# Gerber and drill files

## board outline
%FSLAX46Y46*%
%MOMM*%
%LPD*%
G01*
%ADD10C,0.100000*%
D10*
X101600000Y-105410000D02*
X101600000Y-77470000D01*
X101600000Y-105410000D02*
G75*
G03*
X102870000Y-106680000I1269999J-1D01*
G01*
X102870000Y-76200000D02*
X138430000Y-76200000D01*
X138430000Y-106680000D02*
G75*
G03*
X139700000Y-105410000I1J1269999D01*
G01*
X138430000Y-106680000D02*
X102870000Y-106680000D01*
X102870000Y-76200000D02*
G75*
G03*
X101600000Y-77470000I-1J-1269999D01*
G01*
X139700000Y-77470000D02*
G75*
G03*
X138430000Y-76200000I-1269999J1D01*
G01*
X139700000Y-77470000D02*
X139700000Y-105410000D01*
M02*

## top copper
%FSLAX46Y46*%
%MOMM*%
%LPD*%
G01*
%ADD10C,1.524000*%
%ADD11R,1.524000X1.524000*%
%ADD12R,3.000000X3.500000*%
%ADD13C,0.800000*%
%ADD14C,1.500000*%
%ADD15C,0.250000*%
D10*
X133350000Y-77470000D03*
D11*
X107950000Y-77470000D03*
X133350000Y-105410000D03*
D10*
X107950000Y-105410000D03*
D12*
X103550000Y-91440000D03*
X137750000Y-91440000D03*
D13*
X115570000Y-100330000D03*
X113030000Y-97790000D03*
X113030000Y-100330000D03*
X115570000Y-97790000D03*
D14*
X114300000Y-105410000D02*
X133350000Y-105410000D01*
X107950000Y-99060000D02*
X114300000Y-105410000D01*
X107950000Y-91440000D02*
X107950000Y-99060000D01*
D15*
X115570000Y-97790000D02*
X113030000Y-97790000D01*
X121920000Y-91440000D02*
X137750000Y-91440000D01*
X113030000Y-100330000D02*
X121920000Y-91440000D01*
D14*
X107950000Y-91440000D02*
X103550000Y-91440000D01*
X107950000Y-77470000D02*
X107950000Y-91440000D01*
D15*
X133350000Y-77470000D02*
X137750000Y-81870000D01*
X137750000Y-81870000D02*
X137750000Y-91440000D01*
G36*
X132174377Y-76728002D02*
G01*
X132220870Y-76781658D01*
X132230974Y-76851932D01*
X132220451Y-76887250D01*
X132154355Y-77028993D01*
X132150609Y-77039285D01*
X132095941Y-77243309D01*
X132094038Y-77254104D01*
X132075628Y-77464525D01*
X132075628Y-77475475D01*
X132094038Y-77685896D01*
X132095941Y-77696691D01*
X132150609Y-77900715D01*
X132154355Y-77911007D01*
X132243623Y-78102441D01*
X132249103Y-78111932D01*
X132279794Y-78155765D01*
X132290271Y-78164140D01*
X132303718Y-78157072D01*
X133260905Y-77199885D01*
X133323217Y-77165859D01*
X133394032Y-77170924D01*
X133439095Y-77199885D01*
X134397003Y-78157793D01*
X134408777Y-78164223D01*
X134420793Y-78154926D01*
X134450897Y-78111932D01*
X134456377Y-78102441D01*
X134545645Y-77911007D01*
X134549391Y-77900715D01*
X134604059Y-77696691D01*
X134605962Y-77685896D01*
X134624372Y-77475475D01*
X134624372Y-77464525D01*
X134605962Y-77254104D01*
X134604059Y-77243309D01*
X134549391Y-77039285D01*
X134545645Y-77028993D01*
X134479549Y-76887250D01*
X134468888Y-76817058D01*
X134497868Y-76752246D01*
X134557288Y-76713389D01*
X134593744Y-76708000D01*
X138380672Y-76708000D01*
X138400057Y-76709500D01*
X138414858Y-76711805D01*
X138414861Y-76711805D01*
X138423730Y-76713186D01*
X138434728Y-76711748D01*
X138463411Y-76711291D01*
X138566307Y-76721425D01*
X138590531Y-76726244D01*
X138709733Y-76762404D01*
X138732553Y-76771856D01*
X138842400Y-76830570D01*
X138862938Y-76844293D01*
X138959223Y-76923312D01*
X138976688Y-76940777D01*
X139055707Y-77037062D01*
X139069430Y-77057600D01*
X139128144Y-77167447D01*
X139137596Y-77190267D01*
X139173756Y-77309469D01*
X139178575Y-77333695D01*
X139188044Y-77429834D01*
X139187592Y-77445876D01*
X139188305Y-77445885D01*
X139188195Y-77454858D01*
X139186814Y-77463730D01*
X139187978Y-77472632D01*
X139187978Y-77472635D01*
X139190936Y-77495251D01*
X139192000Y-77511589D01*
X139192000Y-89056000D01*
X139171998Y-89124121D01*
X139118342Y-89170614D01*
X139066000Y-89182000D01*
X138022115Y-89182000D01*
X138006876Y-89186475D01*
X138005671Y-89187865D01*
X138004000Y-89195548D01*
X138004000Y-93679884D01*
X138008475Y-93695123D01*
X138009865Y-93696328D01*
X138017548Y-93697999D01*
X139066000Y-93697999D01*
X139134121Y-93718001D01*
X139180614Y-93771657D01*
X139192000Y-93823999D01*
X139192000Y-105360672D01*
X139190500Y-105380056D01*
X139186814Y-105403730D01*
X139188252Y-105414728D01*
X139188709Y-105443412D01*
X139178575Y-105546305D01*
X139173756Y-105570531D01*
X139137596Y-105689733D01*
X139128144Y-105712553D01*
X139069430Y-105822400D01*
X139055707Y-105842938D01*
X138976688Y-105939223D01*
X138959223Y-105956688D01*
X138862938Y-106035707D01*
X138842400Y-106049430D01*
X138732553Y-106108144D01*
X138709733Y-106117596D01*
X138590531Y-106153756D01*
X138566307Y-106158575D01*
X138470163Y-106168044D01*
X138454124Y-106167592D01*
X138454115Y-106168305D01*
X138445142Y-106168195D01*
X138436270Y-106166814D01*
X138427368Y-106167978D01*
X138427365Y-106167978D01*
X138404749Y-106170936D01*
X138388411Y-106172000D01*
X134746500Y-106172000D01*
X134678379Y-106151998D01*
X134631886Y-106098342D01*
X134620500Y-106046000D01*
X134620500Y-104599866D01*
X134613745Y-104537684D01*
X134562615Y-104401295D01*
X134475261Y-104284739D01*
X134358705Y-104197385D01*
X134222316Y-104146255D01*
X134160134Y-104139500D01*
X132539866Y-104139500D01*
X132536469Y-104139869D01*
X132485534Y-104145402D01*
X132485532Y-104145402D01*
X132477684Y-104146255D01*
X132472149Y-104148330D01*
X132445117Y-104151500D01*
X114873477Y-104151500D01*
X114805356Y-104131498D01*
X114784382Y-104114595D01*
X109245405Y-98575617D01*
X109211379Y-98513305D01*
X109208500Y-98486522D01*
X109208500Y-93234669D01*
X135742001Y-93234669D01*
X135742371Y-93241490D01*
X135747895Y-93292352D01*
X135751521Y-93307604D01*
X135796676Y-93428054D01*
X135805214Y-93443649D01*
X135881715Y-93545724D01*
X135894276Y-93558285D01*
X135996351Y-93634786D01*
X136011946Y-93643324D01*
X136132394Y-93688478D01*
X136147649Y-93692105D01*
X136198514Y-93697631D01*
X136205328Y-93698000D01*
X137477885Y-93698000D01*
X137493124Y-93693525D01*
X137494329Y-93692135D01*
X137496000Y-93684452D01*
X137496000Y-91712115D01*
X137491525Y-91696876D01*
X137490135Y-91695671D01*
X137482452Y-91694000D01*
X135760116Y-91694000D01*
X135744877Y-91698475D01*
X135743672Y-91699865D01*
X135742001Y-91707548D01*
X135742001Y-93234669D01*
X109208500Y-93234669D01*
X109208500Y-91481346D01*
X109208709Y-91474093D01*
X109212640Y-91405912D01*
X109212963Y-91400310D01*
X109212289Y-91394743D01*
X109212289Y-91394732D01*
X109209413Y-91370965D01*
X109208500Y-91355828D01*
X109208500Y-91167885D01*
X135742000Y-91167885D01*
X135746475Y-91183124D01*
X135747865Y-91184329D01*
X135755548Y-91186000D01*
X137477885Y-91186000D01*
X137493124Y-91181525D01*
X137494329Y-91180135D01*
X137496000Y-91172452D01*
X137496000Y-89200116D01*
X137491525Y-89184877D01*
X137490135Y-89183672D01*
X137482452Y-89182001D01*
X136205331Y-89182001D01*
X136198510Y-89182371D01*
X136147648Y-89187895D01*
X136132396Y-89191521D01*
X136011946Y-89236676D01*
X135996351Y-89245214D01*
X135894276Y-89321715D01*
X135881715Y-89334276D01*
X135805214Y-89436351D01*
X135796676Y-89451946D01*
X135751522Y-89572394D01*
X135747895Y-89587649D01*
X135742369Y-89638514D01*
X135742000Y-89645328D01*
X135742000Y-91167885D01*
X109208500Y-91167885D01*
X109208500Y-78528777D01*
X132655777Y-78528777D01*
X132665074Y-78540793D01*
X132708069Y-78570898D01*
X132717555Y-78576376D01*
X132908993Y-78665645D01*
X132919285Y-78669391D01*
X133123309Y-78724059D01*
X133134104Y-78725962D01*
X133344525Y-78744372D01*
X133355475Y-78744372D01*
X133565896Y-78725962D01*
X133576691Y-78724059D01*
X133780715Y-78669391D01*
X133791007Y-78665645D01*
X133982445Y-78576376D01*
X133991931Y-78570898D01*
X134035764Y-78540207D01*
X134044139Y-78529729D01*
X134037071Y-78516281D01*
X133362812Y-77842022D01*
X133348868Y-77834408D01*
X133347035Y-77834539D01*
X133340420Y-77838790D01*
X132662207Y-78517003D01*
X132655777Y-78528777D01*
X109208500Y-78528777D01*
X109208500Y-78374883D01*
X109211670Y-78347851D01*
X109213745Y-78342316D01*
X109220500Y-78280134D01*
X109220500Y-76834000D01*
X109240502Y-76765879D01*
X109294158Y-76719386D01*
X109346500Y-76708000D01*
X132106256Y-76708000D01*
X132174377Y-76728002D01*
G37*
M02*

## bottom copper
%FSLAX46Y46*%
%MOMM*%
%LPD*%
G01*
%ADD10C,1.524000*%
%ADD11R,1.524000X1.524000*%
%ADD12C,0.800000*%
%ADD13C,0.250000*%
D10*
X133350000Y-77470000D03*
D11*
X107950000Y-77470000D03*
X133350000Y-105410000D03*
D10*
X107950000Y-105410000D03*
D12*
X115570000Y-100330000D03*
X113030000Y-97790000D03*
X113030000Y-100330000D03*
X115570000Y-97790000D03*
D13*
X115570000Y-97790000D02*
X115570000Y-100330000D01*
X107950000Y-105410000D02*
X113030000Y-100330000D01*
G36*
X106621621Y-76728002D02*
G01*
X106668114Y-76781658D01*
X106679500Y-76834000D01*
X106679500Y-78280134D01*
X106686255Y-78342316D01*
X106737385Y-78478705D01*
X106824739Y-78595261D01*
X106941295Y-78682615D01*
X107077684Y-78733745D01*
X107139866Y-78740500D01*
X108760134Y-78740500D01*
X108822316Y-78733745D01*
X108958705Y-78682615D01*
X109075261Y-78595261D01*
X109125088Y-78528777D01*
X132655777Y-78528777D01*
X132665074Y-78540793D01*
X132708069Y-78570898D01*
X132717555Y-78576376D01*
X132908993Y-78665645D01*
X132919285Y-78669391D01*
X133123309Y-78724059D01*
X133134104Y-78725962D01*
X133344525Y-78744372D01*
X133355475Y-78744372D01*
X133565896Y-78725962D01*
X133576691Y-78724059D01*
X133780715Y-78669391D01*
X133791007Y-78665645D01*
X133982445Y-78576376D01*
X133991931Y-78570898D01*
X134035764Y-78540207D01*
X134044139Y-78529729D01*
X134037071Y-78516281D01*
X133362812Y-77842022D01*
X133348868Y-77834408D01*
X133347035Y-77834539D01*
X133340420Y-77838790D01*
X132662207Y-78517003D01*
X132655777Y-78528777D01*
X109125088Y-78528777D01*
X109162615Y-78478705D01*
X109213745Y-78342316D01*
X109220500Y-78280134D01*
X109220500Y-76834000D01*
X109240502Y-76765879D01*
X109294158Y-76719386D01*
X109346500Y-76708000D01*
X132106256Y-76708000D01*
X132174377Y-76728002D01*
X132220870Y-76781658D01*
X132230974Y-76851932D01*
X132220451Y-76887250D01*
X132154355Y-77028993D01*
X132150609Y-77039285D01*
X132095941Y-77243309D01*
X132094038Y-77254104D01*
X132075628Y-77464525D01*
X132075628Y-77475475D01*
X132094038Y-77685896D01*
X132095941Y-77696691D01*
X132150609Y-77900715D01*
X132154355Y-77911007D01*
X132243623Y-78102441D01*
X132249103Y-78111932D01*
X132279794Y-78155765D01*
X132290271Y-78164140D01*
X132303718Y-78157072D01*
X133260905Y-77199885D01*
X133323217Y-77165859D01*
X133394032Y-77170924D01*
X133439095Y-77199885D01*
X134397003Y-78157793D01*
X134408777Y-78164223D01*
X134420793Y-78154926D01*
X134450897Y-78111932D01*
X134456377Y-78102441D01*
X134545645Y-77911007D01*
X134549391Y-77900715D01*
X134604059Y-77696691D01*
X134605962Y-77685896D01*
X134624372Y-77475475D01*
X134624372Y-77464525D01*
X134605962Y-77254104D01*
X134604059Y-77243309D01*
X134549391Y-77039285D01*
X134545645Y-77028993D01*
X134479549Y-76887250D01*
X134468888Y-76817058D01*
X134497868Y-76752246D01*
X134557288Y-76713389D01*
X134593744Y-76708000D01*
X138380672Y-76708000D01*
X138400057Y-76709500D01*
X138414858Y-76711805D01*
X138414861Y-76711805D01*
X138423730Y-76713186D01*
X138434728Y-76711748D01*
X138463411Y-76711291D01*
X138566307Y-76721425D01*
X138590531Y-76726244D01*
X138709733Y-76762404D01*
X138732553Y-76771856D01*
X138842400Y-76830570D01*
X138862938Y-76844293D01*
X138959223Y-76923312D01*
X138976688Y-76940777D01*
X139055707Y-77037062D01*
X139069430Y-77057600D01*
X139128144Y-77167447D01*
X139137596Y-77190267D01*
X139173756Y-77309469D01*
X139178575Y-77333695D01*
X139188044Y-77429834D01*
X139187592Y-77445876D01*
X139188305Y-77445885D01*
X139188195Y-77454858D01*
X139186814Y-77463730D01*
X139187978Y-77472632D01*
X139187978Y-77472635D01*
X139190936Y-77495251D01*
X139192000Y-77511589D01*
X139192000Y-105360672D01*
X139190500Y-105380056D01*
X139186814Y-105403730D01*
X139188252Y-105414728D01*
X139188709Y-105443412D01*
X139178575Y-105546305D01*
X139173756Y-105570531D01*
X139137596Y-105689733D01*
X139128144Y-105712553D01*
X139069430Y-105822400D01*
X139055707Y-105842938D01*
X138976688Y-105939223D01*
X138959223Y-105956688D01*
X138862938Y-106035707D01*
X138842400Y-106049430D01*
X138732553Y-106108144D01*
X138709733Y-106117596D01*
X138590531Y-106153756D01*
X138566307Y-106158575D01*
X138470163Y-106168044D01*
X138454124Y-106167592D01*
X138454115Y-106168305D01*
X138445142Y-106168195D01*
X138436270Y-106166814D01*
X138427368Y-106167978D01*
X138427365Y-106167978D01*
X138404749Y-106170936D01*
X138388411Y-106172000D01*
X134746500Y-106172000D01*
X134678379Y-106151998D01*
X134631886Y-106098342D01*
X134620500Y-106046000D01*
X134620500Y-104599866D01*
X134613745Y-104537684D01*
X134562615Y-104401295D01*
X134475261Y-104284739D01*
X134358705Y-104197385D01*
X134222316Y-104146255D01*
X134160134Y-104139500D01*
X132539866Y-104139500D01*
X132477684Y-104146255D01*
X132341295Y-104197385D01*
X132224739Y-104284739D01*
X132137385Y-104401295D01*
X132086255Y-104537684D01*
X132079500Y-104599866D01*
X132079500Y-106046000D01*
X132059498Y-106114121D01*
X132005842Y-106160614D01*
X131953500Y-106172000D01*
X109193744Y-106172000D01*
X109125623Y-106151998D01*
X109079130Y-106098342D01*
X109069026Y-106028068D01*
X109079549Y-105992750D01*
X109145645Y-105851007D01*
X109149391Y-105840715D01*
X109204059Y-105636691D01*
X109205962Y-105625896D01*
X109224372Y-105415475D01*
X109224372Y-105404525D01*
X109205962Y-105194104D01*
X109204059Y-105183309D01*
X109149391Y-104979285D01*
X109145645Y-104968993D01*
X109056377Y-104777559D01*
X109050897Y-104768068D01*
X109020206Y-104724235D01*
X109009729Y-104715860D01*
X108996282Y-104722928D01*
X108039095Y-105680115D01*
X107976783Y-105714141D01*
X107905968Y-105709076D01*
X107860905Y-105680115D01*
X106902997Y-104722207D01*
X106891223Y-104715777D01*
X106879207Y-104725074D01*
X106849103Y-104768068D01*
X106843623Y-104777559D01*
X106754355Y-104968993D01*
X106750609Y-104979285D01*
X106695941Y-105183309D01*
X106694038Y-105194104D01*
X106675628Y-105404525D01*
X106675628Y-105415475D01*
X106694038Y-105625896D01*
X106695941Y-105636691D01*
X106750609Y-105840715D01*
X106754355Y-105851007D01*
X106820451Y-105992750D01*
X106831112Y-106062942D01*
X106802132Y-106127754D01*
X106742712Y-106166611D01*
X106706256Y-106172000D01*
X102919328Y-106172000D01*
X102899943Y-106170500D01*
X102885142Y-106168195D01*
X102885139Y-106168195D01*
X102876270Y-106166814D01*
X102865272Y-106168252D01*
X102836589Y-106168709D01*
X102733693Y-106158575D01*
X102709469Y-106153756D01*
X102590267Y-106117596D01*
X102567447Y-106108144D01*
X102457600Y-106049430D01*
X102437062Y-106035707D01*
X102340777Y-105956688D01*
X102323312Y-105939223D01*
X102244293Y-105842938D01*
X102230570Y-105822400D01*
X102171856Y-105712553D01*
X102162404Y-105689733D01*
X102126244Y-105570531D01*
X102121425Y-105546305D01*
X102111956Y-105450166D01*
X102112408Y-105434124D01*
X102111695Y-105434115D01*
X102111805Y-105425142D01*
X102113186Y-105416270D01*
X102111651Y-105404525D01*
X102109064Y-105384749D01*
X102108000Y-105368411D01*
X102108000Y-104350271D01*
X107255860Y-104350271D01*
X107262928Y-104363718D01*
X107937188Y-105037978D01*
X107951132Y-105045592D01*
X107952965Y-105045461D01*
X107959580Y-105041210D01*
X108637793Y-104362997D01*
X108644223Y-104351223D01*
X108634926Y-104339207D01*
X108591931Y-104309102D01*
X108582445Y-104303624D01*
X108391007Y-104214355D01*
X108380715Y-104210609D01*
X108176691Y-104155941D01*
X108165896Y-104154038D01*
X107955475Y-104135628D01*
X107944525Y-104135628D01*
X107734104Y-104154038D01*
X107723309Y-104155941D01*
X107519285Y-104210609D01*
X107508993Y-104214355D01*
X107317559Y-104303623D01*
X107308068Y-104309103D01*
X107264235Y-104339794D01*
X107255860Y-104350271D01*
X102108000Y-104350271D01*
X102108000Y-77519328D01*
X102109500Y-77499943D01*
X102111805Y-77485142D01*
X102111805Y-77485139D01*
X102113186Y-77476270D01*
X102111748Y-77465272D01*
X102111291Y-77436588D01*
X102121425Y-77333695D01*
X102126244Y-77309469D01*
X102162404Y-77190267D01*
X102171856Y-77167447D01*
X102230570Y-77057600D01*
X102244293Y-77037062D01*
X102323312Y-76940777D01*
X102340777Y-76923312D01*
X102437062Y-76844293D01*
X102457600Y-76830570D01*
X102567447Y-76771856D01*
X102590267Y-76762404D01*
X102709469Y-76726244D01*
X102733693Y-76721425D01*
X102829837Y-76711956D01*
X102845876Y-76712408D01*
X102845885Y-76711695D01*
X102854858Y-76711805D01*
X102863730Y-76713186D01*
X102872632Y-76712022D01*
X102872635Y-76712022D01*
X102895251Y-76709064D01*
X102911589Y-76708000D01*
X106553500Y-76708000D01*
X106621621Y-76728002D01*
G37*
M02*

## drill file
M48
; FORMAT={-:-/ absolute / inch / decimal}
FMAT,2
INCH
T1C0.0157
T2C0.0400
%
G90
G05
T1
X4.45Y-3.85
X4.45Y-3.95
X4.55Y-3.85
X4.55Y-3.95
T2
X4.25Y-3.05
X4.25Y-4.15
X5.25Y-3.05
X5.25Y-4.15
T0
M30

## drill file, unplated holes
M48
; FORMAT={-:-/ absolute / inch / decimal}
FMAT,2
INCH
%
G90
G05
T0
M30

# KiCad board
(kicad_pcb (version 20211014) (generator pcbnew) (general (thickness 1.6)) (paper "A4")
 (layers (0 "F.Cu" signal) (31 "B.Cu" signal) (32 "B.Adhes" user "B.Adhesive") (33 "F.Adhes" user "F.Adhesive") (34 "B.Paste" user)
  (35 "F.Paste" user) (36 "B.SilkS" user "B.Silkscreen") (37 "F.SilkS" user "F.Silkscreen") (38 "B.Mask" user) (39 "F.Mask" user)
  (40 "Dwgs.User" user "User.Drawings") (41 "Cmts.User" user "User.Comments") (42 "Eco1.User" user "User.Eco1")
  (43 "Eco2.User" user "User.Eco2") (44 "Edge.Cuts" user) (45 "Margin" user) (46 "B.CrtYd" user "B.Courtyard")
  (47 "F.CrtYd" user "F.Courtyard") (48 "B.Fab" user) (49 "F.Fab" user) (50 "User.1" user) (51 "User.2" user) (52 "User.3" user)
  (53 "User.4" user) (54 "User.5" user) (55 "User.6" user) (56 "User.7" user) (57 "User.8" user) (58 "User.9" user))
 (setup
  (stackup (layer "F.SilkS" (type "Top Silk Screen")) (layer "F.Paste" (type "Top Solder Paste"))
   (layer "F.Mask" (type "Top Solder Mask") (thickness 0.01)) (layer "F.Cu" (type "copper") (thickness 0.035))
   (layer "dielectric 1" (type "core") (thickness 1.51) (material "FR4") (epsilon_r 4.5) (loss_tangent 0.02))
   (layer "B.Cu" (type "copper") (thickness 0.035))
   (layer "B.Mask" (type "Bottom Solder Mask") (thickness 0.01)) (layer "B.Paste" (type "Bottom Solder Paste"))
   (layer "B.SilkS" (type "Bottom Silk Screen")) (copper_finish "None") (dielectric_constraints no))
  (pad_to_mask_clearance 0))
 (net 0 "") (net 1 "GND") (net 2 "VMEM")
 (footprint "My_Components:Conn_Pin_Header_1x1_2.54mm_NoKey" (layer "F.Cu") (at 133.35 77.47)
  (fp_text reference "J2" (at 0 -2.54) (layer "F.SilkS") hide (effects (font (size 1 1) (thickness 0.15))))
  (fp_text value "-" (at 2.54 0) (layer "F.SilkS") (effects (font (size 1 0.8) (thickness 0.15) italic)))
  (pad "1" thru_hole circle locked (at 0 0) (size 1.524 1.524) (drill 1.016) (layers *.Cu *.Mask) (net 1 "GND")))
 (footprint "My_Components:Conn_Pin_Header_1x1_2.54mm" (layer "F.Cu") (at 107.95 77.47)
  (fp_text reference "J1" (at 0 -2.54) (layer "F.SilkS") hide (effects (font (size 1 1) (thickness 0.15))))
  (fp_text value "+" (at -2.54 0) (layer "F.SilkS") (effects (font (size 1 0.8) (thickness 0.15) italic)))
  (pad "1" thru_hole rect locked (at 0 0) (size 1.524 1.524) (drill 1.016) (layers *.Cu *.Mask) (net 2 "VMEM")))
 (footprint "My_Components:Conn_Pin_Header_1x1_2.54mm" (layer "F.Cu") (at 133.35 105.41)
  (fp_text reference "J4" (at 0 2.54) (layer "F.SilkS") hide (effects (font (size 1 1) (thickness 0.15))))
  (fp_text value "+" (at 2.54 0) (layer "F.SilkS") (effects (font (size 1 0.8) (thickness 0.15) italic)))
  (pad "1" thru_hole rect locked (at 0 0) (size 1.524 1.524) (drill 1.016) (layers *.Cu *.Mask) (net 2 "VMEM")))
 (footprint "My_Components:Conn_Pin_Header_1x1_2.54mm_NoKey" (layer "F.Cu") (at 107.95 105.41)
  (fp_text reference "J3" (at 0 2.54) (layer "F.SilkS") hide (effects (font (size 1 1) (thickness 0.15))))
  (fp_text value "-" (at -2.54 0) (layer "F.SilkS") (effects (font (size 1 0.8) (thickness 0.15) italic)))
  (pad "1" thru_hole circle locked (at 0 0) (size 1.524 1.524) (drill 1.016) (layers *.Cu *.Mask) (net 1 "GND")))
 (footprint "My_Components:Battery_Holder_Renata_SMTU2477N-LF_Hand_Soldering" (layer "F.Cu") (at 120.65 91.44)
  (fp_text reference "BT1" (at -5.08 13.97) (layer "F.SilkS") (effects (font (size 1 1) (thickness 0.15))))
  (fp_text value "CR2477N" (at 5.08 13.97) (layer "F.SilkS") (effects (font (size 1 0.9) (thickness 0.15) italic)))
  (pad "1" smd rect (at -17.1 0) (size 3 3.5) (layers "F.Cu" "F.Paste" "F.Mask") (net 2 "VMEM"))
  (pad "2" smd rect (at 17.1 0) (size 3 3.5) (layers "F.Cu" "F.Paste" "F.Mask") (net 1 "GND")))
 (gr_line (start 101.6 105.41) (end 101.6 77.47) (layer "Edge.Cuts") (width 0.1))
 (gr_arc (start 102.87 106.68) (mid 101.971974 106.308026) (end 101.6 105.41) (layer "Edge.Cuts") (width 0.1))
 (gr_line (start 102.87 76.2) (end 138.43 76.2) (layer "Edge.Cuts") (width 0.1))
 (gr_arc (start 139.7 105.41) (mid 139.328026 106.308026) (end 138.43 106.68) (layer "Edge.Cuts") (width 0.1))
 (gr_line (start 138.43 106.68) (end 102.87 106.68) (layer "Edge.Cuts") (width 0.1))
 (gr_arc (start 101.6 77.47) (mid 101.971974 76.571974) (end 102.87 76.2) (layer "Edge.Cuts") (width 0.1))
 (gr_arc (start 138.43 76.2) (mid 139.328026 76.571974) (end 139.7 77.47) (layer "Edge.Cuts") (width 0.1))
 (gr_line (start 139.7 77.47) (end 139.7 105.41) (layer "Edge.Cuts") (width 0.1))
 (segment (start 107.95 91.44) (end 107.95 99.06) (width 1.5) (layer "F.Cu") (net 2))
 (segment (start 107.95 91.44) (end 103.55 91.44) (width 1.5) (layer "F.Cu") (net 2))
 (segment (start 107.95 77.47) (end 107.95 91.44) (width 1.5) (layer "F.Cu") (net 2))
 (segment (start 107.95 99.06) (end 114.3 105.41) (width 1.5) (layer "F.Cu") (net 2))
 (segment (start 114.3 105.41) (end 133.35 105.41) (width 1.5) (layer "F.Cu") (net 2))
 (segment (start 133.35 77.47) (end 137.75 81.87) (width 0.25) (layer "F.Cu") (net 1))
 (segment (start 115.57 97.79) (end 113.03 97.79) (width 0.25) (layer "F.Cu") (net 1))
 (segment (start 121.92 91.44) (end 137.75 91.44) (width 0.25) (layer "F.Cu") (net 1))
 (segment (start 113.03 100.33) (end 121.92 91.44) (width 0.25) (layer "F.Cu") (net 1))
 (segment (start 137.75 81.87) (end 137.75 91.44) (width 0.25) (layer "F.Cu") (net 1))
 (via (at 115.57 100.33) (size 0.8) (drill 0.4) (layers "F.Cu" "B.Cu") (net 1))
 (via (at 113.03 97.79) (size 0.8) (drill 0.4) (layers "F.Cu" "B.Cu") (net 1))
 (via (at 113.03 100.33) (size 0.8) (drill 0.4) (layers "F.Cu" "B.Cu") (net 1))
 (via (at 115.57 97.79) (size 0.8) (drill 0.4) (layers "F.Cu" "B.Cu") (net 1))
 (segment (start 115.57 97.79) (end 115.57 100.33) (width 0.25) (layer "B.Cu") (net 1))
 (segment (start 107.95 105.41) (end 113.03 100.33) (width 0.25) (layer "B.Cu") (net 1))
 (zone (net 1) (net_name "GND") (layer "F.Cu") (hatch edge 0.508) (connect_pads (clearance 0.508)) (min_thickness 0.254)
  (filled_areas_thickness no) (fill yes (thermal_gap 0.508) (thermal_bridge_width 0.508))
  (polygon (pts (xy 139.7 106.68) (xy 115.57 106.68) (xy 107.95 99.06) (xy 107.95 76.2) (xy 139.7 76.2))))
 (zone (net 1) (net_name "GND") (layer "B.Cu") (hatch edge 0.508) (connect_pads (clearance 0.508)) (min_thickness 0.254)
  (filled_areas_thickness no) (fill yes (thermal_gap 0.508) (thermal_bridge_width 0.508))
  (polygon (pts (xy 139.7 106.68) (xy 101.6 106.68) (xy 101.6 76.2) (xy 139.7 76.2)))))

